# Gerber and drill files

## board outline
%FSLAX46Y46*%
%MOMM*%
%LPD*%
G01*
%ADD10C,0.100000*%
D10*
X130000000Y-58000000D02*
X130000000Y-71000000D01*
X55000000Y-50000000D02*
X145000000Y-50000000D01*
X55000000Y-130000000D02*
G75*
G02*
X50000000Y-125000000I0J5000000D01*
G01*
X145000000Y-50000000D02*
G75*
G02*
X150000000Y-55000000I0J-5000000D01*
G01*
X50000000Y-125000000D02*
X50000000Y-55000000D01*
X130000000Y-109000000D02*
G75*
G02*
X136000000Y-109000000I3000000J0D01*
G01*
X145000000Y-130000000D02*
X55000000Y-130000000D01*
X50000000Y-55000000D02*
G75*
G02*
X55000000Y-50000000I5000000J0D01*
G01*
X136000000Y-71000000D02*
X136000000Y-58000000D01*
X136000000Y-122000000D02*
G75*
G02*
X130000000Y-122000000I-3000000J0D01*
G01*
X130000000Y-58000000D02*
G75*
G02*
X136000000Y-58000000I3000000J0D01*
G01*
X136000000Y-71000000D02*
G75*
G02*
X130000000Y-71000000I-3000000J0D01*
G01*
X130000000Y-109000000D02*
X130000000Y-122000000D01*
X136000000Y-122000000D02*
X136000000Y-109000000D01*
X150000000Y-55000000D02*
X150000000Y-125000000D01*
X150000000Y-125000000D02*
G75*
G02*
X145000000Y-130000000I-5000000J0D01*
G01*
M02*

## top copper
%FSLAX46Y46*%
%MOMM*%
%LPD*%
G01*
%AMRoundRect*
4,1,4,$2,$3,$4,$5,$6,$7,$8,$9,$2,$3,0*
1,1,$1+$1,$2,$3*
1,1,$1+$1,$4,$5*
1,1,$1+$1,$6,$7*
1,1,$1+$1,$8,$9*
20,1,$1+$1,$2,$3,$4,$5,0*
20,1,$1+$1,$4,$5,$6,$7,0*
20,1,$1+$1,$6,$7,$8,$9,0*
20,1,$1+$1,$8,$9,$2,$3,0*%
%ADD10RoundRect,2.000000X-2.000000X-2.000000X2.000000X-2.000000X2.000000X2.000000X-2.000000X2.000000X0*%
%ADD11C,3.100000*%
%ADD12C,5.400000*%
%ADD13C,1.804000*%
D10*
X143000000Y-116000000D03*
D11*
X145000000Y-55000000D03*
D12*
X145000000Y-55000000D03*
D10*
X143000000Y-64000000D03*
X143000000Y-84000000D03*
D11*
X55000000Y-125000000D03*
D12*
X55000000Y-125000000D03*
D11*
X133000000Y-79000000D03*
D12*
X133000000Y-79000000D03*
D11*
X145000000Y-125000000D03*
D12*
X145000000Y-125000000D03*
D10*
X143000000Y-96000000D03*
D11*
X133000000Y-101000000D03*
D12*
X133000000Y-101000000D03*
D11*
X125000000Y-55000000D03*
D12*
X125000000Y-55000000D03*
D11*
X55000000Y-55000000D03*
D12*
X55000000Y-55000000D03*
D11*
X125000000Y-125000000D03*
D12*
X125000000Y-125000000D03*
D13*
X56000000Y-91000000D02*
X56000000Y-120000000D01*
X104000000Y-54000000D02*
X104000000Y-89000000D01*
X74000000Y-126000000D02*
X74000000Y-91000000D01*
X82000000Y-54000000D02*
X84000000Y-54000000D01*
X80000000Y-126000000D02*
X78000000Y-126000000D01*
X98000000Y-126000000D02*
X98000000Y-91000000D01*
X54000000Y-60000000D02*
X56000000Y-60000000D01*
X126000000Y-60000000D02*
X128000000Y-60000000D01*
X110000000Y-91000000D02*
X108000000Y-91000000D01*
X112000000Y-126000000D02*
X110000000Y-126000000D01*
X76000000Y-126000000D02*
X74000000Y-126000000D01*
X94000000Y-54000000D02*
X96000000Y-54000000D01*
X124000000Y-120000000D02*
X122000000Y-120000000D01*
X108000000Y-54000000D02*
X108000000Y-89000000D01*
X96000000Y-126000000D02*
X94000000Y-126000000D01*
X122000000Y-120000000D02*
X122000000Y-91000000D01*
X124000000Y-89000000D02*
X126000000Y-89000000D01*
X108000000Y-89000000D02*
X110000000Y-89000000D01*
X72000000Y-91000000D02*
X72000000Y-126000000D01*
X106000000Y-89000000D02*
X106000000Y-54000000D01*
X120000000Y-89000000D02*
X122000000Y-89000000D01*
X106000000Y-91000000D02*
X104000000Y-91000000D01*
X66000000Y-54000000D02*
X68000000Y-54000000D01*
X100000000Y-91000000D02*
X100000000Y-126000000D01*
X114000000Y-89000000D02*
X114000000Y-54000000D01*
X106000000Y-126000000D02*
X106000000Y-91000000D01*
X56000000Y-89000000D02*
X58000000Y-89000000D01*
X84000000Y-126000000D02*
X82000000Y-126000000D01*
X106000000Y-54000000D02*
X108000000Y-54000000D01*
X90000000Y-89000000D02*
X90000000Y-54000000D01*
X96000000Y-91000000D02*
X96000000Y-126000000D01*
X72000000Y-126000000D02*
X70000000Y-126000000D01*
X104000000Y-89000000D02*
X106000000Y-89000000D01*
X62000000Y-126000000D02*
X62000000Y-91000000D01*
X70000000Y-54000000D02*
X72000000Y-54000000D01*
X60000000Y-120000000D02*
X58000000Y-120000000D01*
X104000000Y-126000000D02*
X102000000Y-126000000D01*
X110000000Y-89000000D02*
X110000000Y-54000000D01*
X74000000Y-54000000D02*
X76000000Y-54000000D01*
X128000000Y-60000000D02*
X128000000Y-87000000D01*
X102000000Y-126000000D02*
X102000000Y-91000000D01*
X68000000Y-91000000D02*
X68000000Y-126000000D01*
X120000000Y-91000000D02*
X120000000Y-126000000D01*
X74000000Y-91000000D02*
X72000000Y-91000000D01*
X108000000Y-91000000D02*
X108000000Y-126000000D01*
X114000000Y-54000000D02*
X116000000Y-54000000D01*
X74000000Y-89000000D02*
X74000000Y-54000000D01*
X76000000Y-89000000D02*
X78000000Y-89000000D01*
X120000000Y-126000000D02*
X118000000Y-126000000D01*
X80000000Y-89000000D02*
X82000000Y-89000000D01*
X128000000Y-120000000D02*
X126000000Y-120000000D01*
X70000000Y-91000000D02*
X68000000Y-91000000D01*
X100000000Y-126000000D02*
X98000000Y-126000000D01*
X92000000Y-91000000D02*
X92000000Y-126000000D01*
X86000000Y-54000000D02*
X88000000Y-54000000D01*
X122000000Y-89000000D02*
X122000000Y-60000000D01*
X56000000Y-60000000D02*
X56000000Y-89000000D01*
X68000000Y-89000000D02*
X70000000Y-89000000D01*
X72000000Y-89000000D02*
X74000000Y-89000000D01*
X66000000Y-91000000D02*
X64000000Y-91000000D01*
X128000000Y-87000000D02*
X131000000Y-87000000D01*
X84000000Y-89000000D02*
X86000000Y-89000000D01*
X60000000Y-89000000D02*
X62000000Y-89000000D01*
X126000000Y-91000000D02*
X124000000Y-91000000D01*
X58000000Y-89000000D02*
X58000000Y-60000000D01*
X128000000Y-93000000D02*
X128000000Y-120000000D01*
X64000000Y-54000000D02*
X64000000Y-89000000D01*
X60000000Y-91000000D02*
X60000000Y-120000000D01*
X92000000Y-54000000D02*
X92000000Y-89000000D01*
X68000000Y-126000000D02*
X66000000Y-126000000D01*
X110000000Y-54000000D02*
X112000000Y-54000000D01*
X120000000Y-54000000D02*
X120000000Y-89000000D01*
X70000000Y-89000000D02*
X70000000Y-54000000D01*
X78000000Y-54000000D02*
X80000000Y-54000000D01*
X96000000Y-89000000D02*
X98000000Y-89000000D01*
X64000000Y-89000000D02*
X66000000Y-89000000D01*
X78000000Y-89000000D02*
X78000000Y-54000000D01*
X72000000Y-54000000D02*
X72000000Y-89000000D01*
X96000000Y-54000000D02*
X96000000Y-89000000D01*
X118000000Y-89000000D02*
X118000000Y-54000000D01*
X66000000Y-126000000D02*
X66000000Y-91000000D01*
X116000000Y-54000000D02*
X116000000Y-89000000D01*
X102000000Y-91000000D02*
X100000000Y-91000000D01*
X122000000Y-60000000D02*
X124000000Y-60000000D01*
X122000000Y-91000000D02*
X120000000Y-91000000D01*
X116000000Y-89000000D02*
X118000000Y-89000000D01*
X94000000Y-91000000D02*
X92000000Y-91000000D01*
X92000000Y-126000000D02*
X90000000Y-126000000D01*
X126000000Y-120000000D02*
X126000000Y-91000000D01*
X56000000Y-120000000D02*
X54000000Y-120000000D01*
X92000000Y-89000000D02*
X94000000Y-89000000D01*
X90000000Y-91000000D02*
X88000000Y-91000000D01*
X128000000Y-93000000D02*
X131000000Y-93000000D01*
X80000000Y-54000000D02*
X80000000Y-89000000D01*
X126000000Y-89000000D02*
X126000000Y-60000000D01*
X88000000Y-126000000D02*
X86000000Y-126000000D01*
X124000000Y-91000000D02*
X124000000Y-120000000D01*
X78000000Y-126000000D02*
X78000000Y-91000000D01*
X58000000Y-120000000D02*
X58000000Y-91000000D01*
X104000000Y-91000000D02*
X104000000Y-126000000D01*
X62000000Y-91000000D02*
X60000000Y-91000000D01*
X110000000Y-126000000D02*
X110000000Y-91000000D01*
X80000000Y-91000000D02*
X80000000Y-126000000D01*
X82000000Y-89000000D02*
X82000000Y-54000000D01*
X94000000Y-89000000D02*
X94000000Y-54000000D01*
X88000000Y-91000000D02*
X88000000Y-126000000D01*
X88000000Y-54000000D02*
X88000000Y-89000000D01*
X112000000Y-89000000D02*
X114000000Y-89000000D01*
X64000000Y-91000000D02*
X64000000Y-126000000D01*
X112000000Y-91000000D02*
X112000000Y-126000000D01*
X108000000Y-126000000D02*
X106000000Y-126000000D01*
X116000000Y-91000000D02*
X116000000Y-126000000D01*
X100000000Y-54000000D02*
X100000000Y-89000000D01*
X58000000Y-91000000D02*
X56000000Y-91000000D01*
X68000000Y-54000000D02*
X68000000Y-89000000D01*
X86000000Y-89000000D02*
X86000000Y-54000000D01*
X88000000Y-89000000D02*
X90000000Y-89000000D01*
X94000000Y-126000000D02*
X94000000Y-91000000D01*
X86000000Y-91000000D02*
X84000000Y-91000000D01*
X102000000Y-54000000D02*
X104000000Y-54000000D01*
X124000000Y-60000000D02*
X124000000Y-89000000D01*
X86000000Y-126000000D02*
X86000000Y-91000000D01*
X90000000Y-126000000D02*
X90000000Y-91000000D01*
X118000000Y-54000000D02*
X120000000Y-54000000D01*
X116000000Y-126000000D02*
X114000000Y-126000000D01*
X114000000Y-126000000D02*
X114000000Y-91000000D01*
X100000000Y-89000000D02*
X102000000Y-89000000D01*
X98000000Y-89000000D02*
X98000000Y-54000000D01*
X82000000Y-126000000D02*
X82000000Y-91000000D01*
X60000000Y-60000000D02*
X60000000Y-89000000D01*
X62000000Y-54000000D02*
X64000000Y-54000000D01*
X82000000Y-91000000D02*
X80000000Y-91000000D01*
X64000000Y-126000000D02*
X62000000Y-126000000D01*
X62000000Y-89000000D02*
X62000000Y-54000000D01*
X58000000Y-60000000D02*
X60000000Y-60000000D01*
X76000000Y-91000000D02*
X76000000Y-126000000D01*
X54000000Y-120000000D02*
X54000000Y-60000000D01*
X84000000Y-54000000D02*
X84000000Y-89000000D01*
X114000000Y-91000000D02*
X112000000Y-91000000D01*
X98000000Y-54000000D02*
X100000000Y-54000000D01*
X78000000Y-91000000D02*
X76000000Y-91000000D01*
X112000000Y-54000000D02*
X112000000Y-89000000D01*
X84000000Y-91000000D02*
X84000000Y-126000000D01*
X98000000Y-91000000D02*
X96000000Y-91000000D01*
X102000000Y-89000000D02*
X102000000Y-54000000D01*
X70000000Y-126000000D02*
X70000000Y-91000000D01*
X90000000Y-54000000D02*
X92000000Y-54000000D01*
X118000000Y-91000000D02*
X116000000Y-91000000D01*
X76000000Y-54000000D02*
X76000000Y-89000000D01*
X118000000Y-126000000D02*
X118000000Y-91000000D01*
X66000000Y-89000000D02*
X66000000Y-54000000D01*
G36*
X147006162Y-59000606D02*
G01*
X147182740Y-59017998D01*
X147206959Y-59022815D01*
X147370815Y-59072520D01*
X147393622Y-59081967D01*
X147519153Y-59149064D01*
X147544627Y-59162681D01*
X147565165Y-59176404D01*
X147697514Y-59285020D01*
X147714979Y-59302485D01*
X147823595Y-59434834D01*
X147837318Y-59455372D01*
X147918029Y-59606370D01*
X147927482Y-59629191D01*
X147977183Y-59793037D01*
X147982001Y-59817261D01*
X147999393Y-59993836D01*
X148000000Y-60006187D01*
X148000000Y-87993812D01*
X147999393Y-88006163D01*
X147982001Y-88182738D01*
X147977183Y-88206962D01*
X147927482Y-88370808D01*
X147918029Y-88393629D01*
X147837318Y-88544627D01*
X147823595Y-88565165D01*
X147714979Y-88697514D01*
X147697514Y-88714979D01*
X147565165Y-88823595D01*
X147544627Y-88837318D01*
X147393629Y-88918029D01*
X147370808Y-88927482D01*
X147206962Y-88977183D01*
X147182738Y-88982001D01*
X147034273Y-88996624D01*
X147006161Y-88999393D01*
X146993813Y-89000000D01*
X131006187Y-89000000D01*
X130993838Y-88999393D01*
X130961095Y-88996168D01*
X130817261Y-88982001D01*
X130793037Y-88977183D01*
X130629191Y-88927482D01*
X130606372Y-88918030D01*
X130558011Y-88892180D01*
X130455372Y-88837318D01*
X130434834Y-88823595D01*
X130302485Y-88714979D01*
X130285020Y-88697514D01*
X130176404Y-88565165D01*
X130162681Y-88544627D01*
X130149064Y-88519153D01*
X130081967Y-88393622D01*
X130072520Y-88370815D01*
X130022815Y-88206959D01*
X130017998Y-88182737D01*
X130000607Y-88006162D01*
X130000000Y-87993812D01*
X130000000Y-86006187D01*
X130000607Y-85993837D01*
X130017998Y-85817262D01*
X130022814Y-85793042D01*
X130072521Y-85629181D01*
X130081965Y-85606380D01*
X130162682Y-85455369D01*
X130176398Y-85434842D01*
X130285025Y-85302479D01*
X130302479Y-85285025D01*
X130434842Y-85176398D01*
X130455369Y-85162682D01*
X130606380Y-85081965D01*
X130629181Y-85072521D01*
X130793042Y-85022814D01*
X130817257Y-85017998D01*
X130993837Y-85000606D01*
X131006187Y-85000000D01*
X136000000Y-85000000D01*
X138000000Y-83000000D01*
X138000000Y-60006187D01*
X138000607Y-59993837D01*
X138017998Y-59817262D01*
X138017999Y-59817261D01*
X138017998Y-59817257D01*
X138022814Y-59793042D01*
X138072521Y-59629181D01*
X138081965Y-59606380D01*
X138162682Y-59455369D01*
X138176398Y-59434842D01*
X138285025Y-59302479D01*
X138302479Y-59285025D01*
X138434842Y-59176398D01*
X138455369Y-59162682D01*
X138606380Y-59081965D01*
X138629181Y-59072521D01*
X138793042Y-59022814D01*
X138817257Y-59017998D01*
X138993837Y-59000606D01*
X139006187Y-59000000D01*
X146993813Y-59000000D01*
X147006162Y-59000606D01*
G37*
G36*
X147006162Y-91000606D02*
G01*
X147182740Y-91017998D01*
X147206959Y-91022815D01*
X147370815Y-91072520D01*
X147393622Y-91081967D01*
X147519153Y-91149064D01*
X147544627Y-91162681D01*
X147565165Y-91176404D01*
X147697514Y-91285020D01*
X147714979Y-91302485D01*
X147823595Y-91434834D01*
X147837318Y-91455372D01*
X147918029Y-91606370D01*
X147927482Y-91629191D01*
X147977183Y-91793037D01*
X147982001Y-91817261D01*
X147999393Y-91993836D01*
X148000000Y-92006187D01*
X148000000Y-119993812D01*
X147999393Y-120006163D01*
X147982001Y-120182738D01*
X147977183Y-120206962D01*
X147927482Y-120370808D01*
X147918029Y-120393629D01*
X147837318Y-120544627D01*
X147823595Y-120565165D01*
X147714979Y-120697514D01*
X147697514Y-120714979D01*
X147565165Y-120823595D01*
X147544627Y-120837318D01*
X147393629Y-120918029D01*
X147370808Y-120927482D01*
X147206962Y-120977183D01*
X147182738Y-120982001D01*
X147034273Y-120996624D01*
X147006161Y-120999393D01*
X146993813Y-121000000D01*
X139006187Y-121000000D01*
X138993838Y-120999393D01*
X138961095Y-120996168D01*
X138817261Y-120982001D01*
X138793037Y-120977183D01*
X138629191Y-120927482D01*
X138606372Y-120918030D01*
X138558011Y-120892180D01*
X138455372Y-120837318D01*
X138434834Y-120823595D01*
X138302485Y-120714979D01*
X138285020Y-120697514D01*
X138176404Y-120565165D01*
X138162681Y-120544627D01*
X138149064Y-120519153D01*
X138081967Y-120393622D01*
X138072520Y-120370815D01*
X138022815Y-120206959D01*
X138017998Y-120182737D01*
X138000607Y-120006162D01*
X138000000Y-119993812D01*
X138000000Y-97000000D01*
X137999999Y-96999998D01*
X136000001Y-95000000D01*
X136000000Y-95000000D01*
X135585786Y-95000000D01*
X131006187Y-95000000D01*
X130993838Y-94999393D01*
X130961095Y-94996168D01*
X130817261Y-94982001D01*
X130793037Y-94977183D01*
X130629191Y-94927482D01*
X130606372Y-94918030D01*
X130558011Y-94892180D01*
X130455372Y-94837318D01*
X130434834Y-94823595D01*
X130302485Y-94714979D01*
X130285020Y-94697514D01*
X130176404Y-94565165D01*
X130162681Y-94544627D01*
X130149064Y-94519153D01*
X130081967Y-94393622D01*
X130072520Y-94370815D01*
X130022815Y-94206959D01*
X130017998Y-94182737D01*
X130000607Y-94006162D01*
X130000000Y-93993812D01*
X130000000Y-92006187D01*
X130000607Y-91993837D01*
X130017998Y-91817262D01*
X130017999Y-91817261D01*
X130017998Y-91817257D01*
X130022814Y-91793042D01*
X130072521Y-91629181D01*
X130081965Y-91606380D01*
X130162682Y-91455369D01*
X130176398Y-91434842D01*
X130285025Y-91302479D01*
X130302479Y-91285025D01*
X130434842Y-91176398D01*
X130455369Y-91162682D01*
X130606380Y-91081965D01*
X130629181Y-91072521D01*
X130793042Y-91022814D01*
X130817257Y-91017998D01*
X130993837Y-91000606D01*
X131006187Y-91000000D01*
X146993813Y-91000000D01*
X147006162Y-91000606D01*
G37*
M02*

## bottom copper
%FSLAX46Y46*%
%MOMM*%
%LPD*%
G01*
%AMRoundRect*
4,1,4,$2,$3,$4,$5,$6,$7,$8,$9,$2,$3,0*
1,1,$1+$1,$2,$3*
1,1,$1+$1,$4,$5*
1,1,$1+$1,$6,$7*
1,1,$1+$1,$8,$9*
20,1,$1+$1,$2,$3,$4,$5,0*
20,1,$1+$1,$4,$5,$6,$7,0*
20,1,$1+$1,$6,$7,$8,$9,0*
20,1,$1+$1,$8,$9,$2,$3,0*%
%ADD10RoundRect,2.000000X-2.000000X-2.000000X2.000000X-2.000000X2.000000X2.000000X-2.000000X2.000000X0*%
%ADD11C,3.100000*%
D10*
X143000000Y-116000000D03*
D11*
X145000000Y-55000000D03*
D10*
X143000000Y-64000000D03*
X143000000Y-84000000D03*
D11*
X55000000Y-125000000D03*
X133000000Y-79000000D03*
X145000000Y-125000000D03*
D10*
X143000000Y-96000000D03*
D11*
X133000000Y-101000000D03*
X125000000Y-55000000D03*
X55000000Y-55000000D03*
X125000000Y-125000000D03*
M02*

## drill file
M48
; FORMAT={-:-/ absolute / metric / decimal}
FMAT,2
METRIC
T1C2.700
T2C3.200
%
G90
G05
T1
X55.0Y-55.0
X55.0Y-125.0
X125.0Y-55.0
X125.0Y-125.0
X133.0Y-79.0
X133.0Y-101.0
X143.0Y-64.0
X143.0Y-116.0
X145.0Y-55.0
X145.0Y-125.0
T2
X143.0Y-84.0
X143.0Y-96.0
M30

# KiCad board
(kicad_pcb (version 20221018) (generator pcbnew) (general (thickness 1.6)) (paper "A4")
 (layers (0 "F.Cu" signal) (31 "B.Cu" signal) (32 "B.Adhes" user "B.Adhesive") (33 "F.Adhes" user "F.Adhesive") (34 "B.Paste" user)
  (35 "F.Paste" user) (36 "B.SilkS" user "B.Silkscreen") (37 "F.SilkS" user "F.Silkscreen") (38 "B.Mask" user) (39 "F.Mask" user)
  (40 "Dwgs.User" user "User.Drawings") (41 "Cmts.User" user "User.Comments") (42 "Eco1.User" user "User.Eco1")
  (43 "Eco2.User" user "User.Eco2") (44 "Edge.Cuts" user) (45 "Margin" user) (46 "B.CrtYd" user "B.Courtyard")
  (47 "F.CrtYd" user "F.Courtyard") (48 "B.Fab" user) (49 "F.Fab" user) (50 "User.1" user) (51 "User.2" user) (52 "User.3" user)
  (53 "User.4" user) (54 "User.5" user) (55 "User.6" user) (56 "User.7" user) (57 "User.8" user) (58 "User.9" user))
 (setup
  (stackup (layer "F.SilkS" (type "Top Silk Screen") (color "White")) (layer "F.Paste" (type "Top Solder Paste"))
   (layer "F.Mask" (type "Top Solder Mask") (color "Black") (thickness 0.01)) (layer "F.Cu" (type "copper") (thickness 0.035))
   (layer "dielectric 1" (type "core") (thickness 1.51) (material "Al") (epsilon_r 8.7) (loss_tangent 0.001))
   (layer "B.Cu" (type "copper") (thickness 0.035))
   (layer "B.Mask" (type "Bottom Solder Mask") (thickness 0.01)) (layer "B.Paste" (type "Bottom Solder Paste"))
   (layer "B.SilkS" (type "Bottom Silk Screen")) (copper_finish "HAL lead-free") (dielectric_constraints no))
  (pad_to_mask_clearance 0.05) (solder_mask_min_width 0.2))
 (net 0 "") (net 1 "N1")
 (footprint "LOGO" (layer "F.Cu") (at 117 114)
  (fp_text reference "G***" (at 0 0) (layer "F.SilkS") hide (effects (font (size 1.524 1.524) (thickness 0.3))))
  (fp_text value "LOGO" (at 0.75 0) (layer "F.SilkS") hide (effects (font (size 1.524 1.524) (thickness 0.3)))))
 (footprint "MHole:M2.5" (layer "F.Cu") (at 143 116)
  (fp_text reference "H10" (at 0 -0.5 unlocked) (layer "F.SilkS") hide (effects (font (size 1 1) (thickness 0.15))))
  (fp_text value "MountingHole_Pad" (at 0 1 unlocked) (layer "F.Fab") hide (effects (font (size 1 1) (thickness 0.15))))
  (pad "1" thru_hole roundrect (at 0 0) (size 8 8) (drill 2.7) (layers "*.Cu" "*.Mask") (roundrect_rratio 0.25) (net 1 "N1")))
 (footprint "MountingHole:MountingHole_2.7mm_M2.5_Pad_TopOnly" (layer "F.Cu") (at 145 55)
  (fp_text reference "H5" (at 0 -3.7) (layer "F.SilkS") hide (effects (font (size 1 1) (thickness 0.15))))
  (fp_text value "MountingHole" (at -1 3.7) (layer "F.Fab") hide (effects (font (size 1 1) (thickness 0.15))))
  (pad "1" thru_hole circle (at 0 0) (size 3.1 3.1) (drill 2.7) (layers "*.Cu" "*.Mask"))
  (pad "1" connect circle (at 0 0) (size 5.4 5.4) (layers "F.Cu" "F.Mask")))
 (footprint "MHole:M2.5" (layer "F.Cu") (at 143 64)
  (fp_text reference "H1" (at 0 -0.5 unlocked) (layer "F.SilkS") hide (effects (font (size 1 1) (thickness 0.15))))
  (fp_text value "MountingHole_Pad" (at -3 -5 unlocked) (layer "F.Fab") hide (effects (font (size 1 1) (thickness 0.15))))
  (pad "1" thru_hole roundrect (at 0 0) (size 8 8) (drill 2.7) (layers "*.Cu" "*.Mask") (roundrect_rratio 0.25) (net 1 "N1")))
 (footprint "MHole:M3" (layer "F.Cu") (at 143 84)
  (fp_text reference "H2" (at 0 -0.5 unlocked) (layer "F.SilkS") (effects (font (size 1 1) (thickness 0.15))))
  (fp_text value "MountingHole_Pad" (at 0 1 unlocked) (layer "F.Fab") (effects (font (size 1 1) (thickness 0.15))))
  (pad "1" thru_hole roundrect (at 0 0) (size 8 8) (drill 3.2) (layers "*.Cu" "*.Mask") (roundrect_rratio 0.25) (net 1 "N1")))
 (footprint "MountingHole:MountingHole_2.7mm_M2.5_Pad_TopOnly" (layer "F.Cu") (at 55 125)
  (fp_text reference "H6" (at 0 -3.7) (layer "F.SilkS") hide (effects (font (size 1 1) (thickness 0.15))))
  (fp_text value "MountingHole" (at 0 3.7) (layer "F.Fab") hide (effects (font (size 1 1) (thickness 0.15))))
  (pad "1" thru_hole circle (at 0 0) (size 3.1 3.1) (drill 2.7) (layers "*.Cu" "*.Mask"))
  (pad "1" connect circle (at 0 0) (size 5.4 5.4) (layers "F.Cu" "F.Mask")))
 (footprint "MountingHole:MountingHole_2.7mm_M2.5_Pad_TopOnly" (layer "F.Cu") (at 133 79)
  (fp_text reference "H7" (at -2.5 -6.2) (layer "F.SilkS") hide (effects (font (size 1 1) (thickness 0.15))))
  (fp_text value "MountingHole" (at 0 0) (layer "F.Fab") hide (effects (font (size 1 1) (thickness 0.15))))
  (pad "1" thru_hole circle (at 0 0) (size 3.1 3.1) (drill 2.7) (layers "*.Cu" "*.Mask"))
  (pad "1" connect circle (at 0 0) (size 5.4 5.4) (layers "F.Cu" "F.Mask")))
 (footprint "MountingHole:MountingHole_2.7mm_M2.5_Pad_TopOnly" (layer "F.Cu") (at 145 125)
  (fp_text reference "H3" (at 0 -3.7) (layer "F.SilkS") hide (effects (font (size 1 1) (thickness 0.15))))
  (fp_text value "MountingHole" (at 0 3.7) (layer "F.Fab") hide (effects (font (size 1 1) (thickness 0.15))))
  (pad "1" thru_hole circle (at 0 0) (size 3.1 3.1) (drill 2.7) (layers "*.Cu" "*.Mask"))
  (pad "1" connect circle (at 0 0) (size 5.4 5.4) (layers "F.Cu" "F.Mask")))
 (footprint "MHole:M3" (layer "F.Cu") (at 143 96)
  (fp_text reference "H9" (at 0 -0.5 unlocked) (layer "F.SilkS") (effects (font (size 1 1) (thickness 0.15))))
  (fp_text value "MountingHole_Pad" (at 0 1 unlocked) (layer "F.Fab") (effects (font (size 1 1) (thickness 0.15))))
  (pad "1" thru_hole roundrect (at 0 0) (size 8 8) (drill 3.2) (layers "*.Cu" "*.Mask") (roundrect_rratio 0.25) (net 1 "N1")))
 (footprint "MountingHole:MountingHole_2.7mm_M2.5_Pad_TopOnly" (layer "F.Cu") (at 133 101)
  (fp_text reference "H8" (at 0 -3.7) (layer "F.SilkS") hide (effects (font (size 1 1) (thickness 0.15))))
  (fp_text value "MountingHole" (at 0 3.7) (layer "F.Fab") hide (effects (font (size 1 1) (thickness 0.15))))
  (pad "1" thru_hole circle (at 0 0) (size 3.1 3.1) (drill 2.7) (layers "*.Cu" "*.Mask"))
  (pad "1" connect circle (at 0 0) (size 5.4 5.4) (layers "F.Cu" "F.Mask")))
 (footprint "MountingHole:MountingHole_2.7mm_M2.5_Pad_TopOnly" (layer "F.Cu") (at 125 55)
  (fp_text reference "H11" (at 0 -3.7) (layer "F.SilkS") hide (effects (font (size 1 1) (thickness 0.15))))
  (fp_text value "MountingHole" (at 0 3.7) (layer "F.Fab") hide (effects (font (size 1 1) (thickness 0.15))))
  (pad "1" thru_hole circle (at 0 0) (size 3.1 3.1) (drill 2.7) (layers "*.Cu" "*.Mask"))
  (pad "1" connect circle (at 0 0) (size 5.4 5.4) (layers "F.Cu" "F.Mask")))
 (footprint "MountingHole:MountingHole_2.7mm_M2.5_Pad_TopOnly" (layer "F.Cu") (at 55 55)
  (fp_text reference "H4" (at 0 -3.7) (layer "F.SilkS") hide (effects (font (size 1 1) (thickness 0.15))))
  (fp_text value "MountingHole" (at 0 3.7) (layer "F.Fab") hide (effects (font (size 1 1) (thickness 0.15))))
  (pad "1" thru_hole circle (at 0 0) (size 3.1 3.1) (drill 2.7) (layers "*.Cu" "*.Mask"))
  (pad "1" connect circle (at 0 0) (size 5.4 5.4) (layers "F.Cu" "F.Mask")))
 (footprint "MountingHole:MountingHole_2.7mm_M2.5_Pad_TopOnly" (layer "F.Cu") (at 125 125)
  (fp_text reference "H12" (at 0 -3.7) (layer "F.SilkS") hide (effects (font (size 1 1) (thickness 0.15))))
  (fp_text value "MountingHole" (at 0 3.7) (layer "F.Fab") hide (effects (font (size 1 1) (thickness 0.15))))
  (pad "1" thru_hole circle (at 0 0) (size 3.1 3.1) (drill 2.7) (layers "*.Cu" "*.Mask"))
  (pad "1" connect circle (at 0 0) (size 5.4 5.4) (layers "F.Cu" "F.Mask")))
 (gr_line (start 130 58) (end 130 71) (stroke (width 0.1) (type solid)) (layer "Edge.Cuts"))
 (gr_line (start 55 50) (end 145 50) (stroke (width 0.1) (type solid)) (layer "Edge.Cuts"))
 (gr_arc (start 55 130) (mid 51.464466 128.535534) (end 50 125) (stroke (width 0.1) (type solid)) (layer "Edge.Cuts"))
 (gr_arc (start 145 50) (mid 148.535534 51.464466) (end 150 55) (stroke (width 0.1) (type solid)) (layer "Edge.Cuts"))
 (gr_line (start 50 125) (end 50 55) (stroke (width 0.1) (type solid)) (layer "Edge.Cuts"))
 (gr_arc (start 130 109) (mid 133 106) (end 136 109) (stroke (width 0.1) (type solid)) (layer "Edge.Cuts"))
 (gr_line (start 145 130) (end 55 130) (stroke (width 0.1) (type solid)) (layer "Edge.Cuts"))
 (gr_arc (start 50 55) (mid 51.464466 51.464466) (end 55 50) (stroke (width 0.1) (type solid)) (layer "Edge.Cuts"))
 (gr_line (start 136 71) (end 136 58) (stroke (width 0.1) (type solid)) (layer "Edge.Cuts"))
 (gr_arc (start 136 122) (mid 133 125) (end 130 122) (stroke (width 0.1) (type solid)) (layer "Edge.Cuts"))
 (gr_arc (start 130 58) (mid 133 55) (end 136 58) (stroke (width 0.1) (type solid)) (layer "Edge.Cuts"))
 (gr_arc (start 136 71) (mid 133 74) (end 130 71) (stroke (width 0.1) (type solid)) (layer "Edge.Cuts"))
 (gr_line (start 130 109) (end 130 122) (stroke (width 0.1) (type solid)) (layer "Edge.Cuts"))
 (gr_line (start 136 122) (end 136 109) (stroke (width 0.1) (type solid)) (layer "Edge.Cuts"))
 (gr_line (start 150 55) (end 150 125) (stroke (width 0.1) (type solid)) (layer "Edge.Cuts"))
 (gr_arc (start 150 125) (mid 148.535534 128.535534) (end 145 130) (stroke (width 0.1) (type solid)) (layer "Edge.Cuts"))
 (segment (start 56 91) (end 56 120) (width 1.804) (layer "F.Cu") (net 1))
 (segment (start 104 54) (end 104 89) (width 1.804) (layer "F.Cu") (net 1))
 (segment (start 74 126) (end 74 91) (width 1.804) (layer "F.Cu") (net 1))
 (segment (start 82 54) (end 84 54) (width 1.804) (layer "F.Cu") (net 1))
 (segment (start 80 126) (end 78 126) (width 1.804) (layer "F.Cu") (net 1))
 (segment (start 98 126) (end 98 91) (width 1.804) (layer "F.Cu") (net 1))
 (segment (start 54 60) (end 56 60) (width 1.804) (layer "F.Cu") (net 1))
 (segment (start 126 60) (end 128 60) (width 1.804) (layer "F.Cu") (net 1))
 (segment (start 110 91) (end 108 91) (width 1.804) (layer "F.Cu") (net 1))
 (segment (start 112 126) (end 110 126) (width 1.804) (layer "F.Cu") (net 1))
 (segment (start 76 126) (end 74 126) (width 1.804) (layer "F.Cu") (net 1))
 (segment (start 94 54) (end 96 54) (width 1.804) (layer "F.Cu") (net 1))
 (segment (start 124 120) (end 122 120) (width 1.804) (layer "F.Cu") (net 1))
 (segment (start 108 54) (end 108 89) (width 1.804) (layer "F.Cu") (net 1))
 (segment (start 96 126) (end 94 126) (width 1.804) (layer "F.Cu") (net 1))
 (segment (start 122 120) (end 122 91) (width 1.804) (layer "F.Cu") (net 1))
 (segment (start 124 89) (end 126 89) (width 1.804) (layer "F.Cu") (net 1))
 (segment (start 108 89) (end 110 89) (width 1.804) (layer "F.Cu") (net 1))
 (segment (start 72 91) (end 72 126) (width 1.804) (layer "F.Cu") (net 1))
 (segment (start 106 89) (end 106 54) (width 1.804) (layer "F.Cu") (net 1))
 (segment (start 120 89) (end 122 89) (width 1.804) (layer "F.Cu") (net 1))
 (segment (start 106 91) (end 104 91) (width 1.804) (layer "F.Cu") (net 1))
 (segment (start 66 54) (end 68 54) (width 1.804) (layer "F.Cu") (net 1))
 (segment (start 100 91) (end 100 126) (width 1.804) (layer "F.Cu") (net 1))
 (segment (start 114 89) (end 114 54) (width 1.804) (layer "F.Cu") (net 1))
 (segment (start 106 126) (end 106 91) (width 1.804) (layer "F.Cu") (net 1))
 (segment (start 56 89) (end 58 89) (width 1.804) (layer "F.Cu") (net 1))
 (segment (start 84 126) (end 82 126) (width 1.804) (layer "F.Cu") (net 1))
 (segment (start 106 54) (end 108 54) (width 1.804) (layer "F.Cu") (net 1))
 (segment (start 90 89) (end 90 54) (width 1.804) (layer "F.Cu") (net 1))
 (segment (start 96 91) (end 96 126) (width 1.804) (layer "F.Cu") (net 1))
 (segment (start 72 126) (end 70 126) (width 1.804) (layer "F.Cu") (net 1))
 (segment (start 104 89) (end 106 89) (width 1.804) (layer "F.Cu") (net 1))
 (segment (start 62 126) (end 62 91) (width 1.804) (layer "F.Cu") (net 1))
 (segment (start 70 54) (end 72 54) (width 1.804) (layer "F.Cu") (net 1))
 (segment (start 60 120) (end 58 120) (width 1.804) (layer "F.Cu") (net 1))
 (segment (start 104 126) (end 102 126) (width 1.804) (layer "F.Cu") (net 1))
 (segment (start 110 89) (end 110 54) (width 1.804) (layer "F.Cu") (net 1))
 (segment (start 74 54) (end 76 54) (width 1.804) (layer "F.Cu") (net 1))
 (segment (start 128 60) (end 128 87) (width 1.804) (layer "F.Cu") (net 1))
 (segment (start 102 126) (end 102 91) (width 1.804) (layer "F.Cu") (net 1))
 (segment (start 68 91) (end 68 126) (width 1.804) (layer "F.Cu") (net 1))
 (segment (start 120 91) (end 120 126) (width 1.804) (layer "F.Cu") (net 1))
 (segment (start 74 91) (end 72 91) (width 1.804) (layer "F.Cu") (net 1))
 (segment (start 108 91) (end 108 126) (width 1.804) (layer "F.Cu") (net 1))
 (segment (start 114 54) (end 116 54) (width 1.804) (layer "F.Cu") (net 1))
 (segment (start 74 89) (end 74 54) (width 1.804) (layer "F.Cu") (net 1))
 (segment (start 76 89) (end 78 89) (width 1.804) (layer "F.Cu") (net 1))
 (segment (start 120 126) (end 118 126) (width 1.804) (layer "F.Cu") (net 1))
 (segment (start 80 89) (end 82 89) (width 1.804) (layer "F.Cu") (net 1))
 (segment (start 128 120) (end 126 120) (width 1.804) (layer "F.Cu") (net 1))
 (segment (start 70 91) (end 68 91) (width 1.804) (layer "F.Cu") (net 1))
 (segment (start 100 126) (end 98 126) (width 1.804) (layer "F.Cu") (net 1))
 (segment (start 92 91) (end 92 126) (width 1.804) (layer "F.Cu") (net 1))
 (segment (start 86 54) (end 88 54) (width 1.804) (layer "F.Cu") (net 1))
 (segment (start 122 89) (end 122 60) (width 1.804) (layer "F.Cu") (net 1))
 (segment (start 56 60) (end 56 89) (width 1.804) (layer "F.Cu") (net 1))
 (segment (start 68 89) (end 70 89) (width 1.804) (layer "F.Cu") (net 1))
 (segment (start 72 89) (end 74 89) (width 1.804) (layer "F.Cu") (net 1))
 (segment (start 66 91) (end 64 91) (width 1.804) (layer "F.Cu") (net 1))
 (segment (start 128 87) (end 131 87) (width 1.804) (layer "F.Cu") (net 1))
 (segment (start 84 89) (end 86 89) (width 1.804) (layer "F.Cu") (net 1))
 (segment (start 60 89) (end 62 89) (width 1.804) (layer "F.Cu") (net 1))
 (segment (start 126 91) (end 124 91) (width 1.804) (layer "F.Cu") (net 1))
 (segment (start 58 89) (end 58 60) (width 1.804) (layer "F.Cu") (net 1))
 (segment (start 128 93) (end 128 120) (width 1.804) (layer "F.Cu") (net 1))
 (segment (start 64 54) (end 64 89) (width 1.804) (layer "F.Cu") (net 1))
 (segment (start 60 91) (end 60 120) (width 1.804) (layer "F.Cu") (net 1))
 (segment (start 92 54) (end 92 89) (width 1.804) (layer "F.Cu") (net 1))
 (segment (start 68 126) (end 66 126) (width 1.804) (layer "F.Cu") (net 1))
 (segment (start 110 54) (end 112 54) (width 1.804) (layer "F.Cu") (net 1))
 (segment (start 120 54) (end 120 89) (width 1.804) (layer "F.Cu") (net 1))
 (segment (start 70 89) (end 70 54) (width 1.804) (layer "F.Cu") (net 1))
 (segment (start 78 54) (end 80 54) (width 1.804) (layer "F.Cu") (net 1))
 (segment (start 96 89) (end 98 89) (width 1.804) (layer "F.Cu") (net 1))
 (segment (start 64 89) (end 66 89) (width 1.804) (layer "F.Cu") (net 1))
 (segment (start 78 89) (end 78 54) (width 1.804) (layer "F.Cu") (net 1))
 (segment (start 72 54) (end 72 89) (width 1.804) (layer "F.Cu") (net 1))
 (segment (start 96 54) (end 96 89) (width 1.804) (layer "F.Cu") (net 1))
 (segment (start 118 89) (end 118 54) (width 1.804) (layer "F.Cu") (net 1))
 (segment (start 66 126) (end 66 91) (width 1.804) (layer "F.Cu") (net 1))
 (segment (start 116 54) (end 116 89) (width 1.804) (layer "F.Cu") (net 1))
 (segment (start 102 91) (end 100 91) (width 1.804) (layer "F.Cu") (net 1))
 (segment (start 122 60) (end 124 60) (width 1.804) (layer "F.Cu") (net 1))
 (segment (start 122 91) (end 120 91) (width 1.804) (layer "F.Cu") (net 1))
 (segment (start 116 89) (end 118 89) (width 1.804) (layer "F.Cu") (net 1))
 (segment (start 94 91) (end 92 91) (width 1.804) (layer "F.Cu") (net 1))
 (segment (start 92 126) (end 90 126) (width 1.804) (layer "F.Cu") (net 1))
 (segment (start 126 120) (end 126 91) (width 1.804) (layer "F.Cu") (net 1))
 (segment (start 56 120) (end 54 120) (width 1.804) (layer "F.Cu") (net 1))
 (segment (start 92 89) (end 94 89) (width 1.804) (layer "F.Cu") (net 1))
 (segment (start 90 91) (end 88 91) (width 1.804) (layer "F.Cu") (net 1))
 (segment (start 128 93) (end 131 93) (width 1.804) (layer "F.Cu") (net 1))
 (segment (start 80 54) (end 80 89) (width 1.804) (layer "F.Cu") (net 1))
 (segment (start 126 89) (end 126 60) (width 1.804) (layer "F.Cu") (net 1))
 (segment (start 88 126) (end 86 126) (width 1.804) (layer "F.Cu") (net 1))
 (segment (start 124 91) (end 124 120) (width 1.804) (layer "F.Cu") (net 1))
 (segment (start 78 126) (end 78 91) (width 1.804) (layer "F.Cu") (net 1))
 (segment (start 58 120) (end 58 91) (width 1.804) (layer "F.Cu") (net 1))
 (segment (start 104 91) (end 104 126) (width 1.804) (layer "F.Cu") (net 1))
 (segment (start 62 91) (end 60 91) (width 1.804) (layer "F.Cu") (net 1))
 (segment (start 110 126) (end 110 91) (width 1.804) (layer "F.Cu") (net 1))
 (segment (start 80 91) (end 80 126) (width 1.804) (layer "F.Cu") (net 1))
 (segment (start 82 89) (end 82 54) (width 1.804) (layer "F.Cu") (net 1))
 (segment (start 94 89) (end 94 54) (width 1.804) (layer "F.Cu") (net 1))
 (segment (start 88 91) (end 88 126) (width 1.804) (layer "F.Cu") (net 1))
 (segment (start 88 54) (end 88 89) (width 1.804) (layer "F.Cu") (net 1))
 (segment (start 112 89) (end 114 89) (width 1.804) (layer "F.Cu") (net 1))
 (segment (start 64 91) (end 64 126) (width 1.804) (layer "F.Cu") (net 1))
 (segment (start 112 91) (end 112 126) (width 1.804) (layer "F.Cu") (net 1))
 (segment (start 108 126) (end 106 126) (width 1.804) (layer "F.Cu") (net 1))
 (segment (start 116 91) (end 116 126) (width 1.804) (layer "F.Cu") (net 1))
 (segment (start 100 54) (end 100 89) (width 1.804) (layer "F.Cu") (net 1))
 (segment (start 58 91) (end 56 91) (width 1.804) (layer "F.Cu") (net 1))
 (segment (start 68 54) (end 68 89) (width 1.804) (layer "F.Cu") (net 1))
 (segment (start 86 89) (end 86 54) (width 1.804) (layer "F.Cu") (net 1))
 (segment (start 88 89) (end 90 89) (width 1.804) (layer "F.Cu") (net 1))
 (segment (start 94 126) (end 94 91) (width 1.804) (layer "F.Cu") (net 1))
 (segment (start 86 91) (end 84 91) (width 1.804) (layer "F.Cu") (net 1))
 (segment (start 102 54) (end 104 54) (width 1.804) (layer "F.Cu") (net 1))
 (segment (start 124 60) (end 124 89) (width 1.804) (layer "F.Cu") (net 1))
 (segment (start 86 126) (end 86 91) (width 1.804) (layer "F.Cu") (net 1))
 (segment (start 90 126) (end 90 91) (width 1.804) (layer "F.Cu") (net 1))
 (segment (start 118 54) (end 120 54) (width 1.804) (layer "F.Cu") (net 1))
 (segment (start 116 126) (end 114 126) (width 1.804) (layer "F.Cu") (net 1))
 (segment (start 114 126) (end 114 91) (width 1.804) (layer "F.Cu") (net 1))
 (segment (start 100 89) (end 102 89) (width 1.804) (layer "F.Cu") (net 1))
 (segment (start 98 89) (end 98 54) (width 1.804) (layer "F.Cu") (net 1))
 (segment (start 82 126) (end 82 91) (width 1.804) (layer "F.Cu") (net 1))
 (segment (start 60 60) (end 60 89) (width 1.804) (layer "F.Cu") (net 1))
 (segment (start 62 54) (end 64 54) (width 1.804) (layer "F.Cu") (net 1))
 (segment (start 82 91) (end 80 91) (width 1.804) (layer "F.Cu") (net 1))
 (segment (start 64 126) (end 62 126) (width 1.804) (layer "F.Cu") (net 1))
 (segment (start 62 89) (end 62 54) (width 1.804) (layer "F.Cu") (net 1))
 (segment (start 58 60) (end 60 60) (width 1.804) (layer "F.Cu") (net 1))
 (segment (start 76 91) (end 76 126) (width 1.804) (layer "F.Cu") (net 1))
 (segment (start 54 120) (end 54 60) (width 1.804) (layer "F.Cu") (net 1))
 (segment (start 84 54) (end 84 89) (width 1.804) (layer "F.Cu") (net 1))
 (segment (start 114 91) (end 112 91) (width 1.804) (layer "F.Cu") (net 1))
 (segment (start 98 54) (end 100 54) (width 1.804) (layer "F.Cu") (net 1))
 (segment (start 78 91) (end 76 91) (width 1.804) (layer "F.Cu") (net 1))
 (segment (start 112 54) (end 112 89) (width 1.804) (layer "F.Cu") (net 1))
 (segment (start 84 91) (end 84 126) (width 1.804) (layer "F.Cu") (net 1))
 (segment (start 98 91) (end 96 91) (width 1.804) (layer "F.Cu") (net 1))
 (segment (start 102 89) (end 102 54) (width 1.804) (layer "F.Cu") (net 1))
 (segment (start 70 126) (end 70 91) (width 1.804) (layer "F.Cu") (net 1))
 (segment (start 90 54) (end 92 54) (width 1.804) (layer "F.Cu") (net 1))
 (segment (start 118 91) (end 116 91) (width 1.804) (layer "F.Cu") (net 1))
 (segment (start 76 54) (end 76 89) (width 1.804) (layer "F.Cu") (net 1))
 (segment (start 118 126) (end 118 91) (width 1.804) (layer "F.Cu") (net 1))
 (segment (start 66 89) (end 66 54) (width 1.804) (layer "F.Cu") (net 1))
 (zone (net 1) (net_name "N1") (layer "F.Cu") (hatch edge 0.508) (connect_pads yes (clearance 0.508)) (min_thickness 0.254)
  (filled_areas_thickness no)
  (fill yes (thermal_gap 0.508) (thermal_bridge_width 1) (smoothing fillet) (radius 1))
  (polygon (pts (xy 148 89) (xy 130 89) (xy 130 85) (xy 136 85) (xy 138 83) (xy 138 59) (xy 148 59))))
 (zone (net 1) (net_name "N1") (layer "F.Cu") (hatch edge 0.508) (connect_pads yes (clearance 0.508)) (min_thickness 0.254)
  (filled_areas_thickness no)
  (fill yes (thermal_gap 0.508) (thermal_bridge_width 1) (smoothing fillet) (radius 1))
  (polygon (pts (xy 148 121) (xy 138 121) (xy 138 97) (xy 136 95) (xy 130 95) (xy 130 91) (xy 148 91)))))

